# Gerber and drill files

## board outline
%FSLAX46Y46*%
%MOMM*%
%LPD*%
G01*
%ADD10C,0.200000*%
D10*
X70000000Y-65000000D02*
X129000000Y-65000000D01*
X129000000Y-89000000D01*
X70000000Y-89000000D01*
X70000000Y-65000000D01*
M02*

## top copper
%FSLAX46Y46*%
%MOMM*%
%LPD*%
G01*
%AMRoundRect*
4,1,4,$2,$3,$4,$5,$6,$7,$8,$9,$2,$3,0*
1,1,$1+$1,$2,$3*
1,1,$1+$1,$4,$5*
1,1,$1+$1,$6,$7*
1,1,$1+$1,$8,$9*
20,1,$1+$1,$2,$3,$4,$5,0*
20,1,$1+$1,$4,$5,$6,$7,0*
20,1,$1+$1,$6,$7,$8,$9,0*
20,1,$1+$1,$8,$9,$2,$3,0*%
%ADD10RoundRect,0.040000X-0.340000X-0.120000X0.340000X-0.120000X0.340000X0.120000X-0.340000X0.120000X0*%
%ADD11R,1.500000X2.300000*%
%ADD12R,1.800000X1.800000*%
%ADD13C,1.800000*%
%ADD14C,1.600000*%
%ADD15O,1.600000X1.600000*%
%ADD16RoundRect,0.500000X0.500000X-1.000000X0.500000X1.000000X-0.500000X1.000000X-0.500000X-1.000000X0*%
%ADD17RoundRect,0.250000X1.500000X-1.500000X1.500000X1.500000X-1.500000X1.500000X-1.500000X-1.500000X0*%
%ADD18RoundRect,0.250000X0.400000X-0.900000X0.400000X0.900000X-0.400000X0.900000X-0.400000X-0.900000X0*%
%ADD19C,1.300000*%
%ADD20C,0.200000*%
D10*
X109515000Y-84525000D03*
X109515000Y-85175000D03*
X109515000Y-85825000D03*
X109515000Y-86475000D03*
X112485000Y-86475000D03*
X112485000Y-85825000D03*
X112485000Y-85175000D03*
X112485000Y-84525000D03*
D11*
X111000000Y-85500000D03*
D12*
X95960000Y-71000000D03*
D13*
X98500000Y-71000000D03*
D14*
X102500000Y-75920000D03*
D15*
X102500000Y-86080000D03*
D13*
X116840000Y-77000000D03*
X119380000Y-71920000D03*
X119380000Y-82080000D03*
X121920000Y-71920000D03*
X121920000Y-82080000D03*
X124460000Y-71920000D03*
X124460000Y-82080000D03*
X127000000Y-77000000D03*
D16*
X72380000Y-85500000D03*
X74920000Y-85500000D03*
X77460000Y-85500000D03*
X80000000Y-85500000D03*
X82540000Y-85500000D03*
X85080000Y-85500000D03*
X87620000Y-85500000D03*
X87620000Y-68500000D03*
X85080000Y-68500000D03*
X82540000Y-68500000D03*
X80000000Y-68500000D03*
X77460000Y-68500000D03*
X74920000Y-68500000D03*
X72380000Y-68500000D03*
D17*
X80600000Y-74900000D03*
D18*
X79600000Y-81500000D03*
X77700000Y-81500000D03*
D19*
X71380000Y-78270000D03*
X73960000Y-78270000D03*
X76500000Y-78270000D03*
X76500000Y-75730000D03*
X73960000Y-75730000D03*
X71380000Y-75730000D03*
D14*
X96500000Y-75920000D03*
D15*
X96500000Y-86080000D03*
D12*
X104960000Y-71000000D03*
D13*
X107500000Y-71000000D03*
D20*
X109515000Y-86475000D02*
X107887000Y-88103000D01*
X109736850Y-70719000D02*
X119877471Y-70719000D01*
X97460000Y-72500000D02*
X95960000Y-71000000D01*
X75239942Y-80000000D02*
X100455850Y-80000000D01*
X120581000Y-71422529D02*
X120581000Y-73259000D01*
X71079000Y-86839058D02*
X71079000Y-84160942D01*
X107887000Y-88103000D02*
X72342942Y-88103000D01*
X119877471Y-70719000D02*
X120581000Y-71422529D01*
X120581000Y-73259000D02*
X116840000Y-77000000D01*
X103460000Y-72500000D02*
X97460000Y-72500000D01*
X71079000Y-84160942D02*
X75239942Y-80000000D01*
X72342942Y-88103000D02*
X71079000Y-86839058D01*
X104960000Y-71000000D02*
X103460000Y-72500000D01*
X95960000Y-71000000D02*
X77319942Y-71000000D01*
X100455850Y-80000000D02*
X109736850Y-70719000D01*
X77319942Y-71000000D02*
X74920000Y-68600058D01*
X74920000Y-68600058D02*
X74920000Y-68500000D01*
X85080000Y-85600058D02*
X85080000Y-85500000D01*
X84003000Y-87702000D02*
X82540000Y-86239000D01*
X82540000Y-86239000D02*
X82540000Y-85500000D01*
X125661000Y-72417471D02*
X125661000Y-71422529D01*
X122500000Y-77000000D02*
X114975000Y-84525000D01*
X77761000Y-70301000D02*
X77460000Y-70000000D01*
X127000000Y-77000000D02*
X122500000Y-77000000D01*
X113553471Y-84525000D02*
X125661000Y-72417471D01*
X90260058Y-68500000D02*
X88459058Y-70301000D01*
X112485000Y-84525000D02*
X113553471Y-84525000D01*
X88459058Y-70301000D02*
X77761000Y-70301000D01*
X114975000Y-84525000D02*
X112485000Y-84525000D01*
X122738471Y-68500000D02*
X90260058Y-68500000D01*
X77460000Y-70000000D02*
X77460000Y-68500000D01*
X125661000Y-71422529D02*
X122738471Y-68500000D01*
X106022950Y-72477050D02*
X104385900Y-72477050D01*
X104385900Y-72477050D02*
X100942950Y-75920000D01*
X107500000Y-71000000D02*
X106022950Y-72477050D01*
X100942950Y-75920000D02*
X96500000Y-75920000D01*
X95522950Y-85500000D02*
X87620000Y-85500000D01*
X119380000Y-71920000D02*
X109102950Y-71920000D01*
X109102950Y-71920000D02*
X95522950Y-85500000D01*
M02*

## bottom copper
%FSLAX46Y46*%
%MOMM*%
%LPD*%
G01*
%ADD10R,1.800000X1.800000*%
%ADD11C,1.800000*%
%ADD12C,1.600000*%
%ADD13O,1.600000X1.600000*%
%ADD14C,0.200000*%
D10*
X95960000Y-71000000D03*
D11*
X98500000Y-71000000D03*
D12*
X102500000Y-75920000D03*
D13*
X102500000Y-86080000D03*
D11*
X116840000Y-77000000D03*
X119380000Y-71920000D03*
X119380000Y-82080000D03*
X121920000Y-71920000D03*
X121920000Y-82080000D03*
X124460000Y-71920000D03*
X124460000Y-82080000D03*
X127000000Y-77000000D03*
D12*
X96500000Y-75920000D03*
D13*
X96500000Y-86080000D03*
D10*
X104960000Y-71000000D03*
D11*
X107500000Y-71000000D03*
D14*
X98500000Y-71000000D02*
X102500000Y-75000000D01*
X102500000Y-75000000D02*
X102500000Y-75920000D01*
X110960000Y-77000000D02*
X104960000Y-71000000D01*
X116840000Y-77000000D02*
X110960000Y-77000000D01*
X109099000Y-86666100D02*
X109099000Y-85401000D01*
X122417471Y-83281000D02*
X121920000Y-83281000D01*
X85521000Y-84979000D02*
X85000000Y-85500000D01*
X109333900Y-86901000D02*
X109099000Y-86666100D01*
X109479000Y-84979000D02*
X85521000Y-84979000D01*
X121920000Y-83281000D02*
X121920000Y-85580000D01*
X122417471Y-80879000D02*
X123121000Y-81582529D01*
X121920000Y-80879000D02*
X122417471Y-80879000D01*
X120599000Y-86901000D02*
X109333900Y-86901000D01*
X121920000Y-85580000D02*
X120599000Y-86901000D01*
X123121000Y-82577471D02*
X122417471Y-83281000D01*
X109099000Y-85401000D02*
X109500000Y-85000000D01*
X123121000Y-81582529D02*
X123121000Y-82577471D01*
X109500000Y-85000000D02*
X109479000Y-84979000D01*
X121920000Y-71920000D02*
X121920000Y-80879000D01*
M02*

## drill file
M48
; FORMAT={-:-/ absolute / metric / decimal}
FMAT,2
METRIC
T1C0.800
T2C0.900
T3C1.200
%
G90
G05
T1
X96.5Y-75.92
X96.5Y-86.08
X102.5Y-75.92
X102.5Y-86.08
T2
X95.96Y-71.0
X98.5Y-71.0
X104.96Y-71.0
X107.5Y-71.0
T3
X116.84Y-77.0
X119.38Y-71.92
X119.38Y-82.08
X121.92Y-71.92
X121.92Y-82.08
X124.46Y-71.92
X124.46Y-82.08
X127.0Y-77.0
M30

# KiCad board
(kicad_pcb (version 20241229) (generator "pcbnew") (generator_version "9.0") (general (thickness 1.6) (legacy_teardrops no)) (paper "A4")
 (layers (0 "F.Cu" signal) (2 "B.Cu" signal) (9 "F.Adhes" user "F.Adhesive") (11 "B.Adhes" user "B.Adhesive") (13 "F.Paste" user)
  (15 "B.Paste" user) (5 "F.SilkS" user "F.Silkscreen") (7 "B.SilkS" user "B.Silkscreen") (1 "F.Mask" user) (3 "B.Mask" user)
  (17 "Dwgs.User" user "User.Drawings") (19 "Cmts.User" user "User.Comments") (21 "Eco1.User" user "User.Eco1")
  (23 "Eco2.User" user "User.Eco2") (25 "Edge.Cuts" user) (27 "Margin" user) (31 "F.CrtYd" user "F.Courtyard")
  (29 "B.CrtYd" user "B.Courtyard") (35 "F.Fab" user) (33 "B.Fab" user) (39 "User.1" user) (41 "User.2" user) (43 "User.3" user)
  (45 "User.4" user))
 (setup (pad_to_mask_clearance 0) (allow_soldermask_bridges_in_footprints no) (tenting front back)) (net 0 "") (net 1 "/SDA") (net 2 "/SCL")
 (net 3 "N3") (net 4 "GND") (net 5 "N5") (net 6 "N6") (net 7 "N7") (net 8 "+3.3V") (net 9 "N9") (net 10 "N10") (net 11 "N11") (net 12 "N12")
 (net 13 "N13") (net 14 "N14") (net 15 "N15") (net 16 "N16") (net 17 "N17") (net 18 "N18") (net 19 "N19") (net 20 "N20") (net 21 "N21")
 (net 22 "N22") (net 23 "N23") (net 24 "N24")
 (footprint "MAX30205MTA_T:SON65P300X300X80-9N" (layer "F.Cu") (at 111 85.5)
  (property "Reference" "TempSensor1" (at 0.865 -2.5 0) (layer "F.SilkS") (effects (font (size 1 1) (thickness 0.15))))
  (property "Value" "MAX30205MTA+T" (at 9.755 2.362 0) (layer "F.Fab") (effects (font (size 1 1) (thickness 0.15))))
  (pad "1" smd roundrect (at -1.485 -0.975) (size 0.76 0.32) (layers "F.Cu" "F.Mask" "F.Paste") (roundrect_rratio 0.125) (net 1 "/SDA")
   (solder_mask_margin 0.102))
  (pad "2" smd roundrect (at -1.485 -0.325) (size 0.76 0.32) (layers "F.Cu" "F.Mask" "F.Paste") (roundrect_rratio 0.125) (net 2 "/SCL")
   (solder_mask_margin 0.102))
  (pad "3" smd roundrect (at -1.485 0.325) (size 0.76 0.32) (layers "F.Cu" "F.Mask" "F.Paste") (roundrect_rratio 0.125) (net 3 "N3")
   (solder_mask_margin 0.102))
  (pad "4" smd roundrect (at -1.485 0.975) (size 0.76 0.32) (layers "F.Cu" "F.Mask" "F.Paste") (roundrect_rratio 0.125) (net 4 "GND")
   (solder_mask_margin 0.102))
  (pad "5" smd roundrect (at 1.485 0.975) (size 0.76 0.32) (layers "F.Cu" "F.Mask" "F.Paste") (roundrect_rratio 0.125) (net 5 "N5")
   (solder_mask_margin 0.102))
  (pad "6" smd roundrect (at 1.485 0.325) (size 0.76 0.32) (layers "F.Cu" "F.Mask" "F.Paste") (roundrect_rratio 0.125) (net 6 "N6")
   (solder_mask_margin 0.102))
  (pad "7" smd roundrect (at 1.485 -0.325) (size 0.76 0.32) (layers "F.Cu" "F.Mask" "F.Paste") (roundrect_rratio 0.125) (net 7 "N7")
   (solder_mask_margin 0.102))
  (pad "8" smd roundrect (at 1.485 -0.975) (size 0.76 0.32) (layers "F.Cu" "F.Mask" "F.Paste") (roundrect_rratio 0.125) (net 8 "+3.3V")
   (solder_mask_margin 0.102))
  (pad "9" smd rect (at 0 0) (size 1.5 2.3) (layers "F.Cu" "F.Mask") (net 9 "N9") (solder_mask_margin 0.102)))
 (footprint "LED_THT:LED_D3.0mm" (layer "F.Cu") (at 95.96 71)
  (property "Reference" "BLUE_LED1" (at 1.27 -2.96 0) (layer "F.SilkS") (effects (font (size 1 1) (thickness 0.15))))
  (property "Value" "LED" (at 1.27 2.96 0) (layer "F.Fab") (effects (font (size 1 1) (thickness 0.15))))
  (pad "1" thru_hole rect (at 0 0) (size 1.8 1.8) (drill 0.9) (layers "*.Cu" "*.Mask") (remove_unused_layers no) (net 4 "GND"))
  (pad "2" thru_hole circle (at 2.54 0) (size 1.8 1.8) (drill 0.9) (layers "*.Cu" "*.Mask") (remove_unused_layers no) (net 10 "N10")))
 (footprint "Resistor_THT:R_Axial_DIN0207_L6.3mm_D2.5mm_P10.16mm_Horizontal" (layer "F.Cu") (at 102.5 75.92 -90)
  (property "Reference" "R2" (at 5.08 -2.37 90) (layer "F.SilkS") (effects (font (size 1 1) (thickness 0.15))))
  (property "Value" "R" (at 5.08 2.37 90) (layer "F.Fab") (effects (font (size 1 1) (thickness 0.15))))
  (pad "1" thru_hole circle (at 0 0 270) (size 1.6 1.6) (drill 0.8) (layers "*.Cu" "*.Mask") (remove_unused_layers no) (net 10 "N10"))
  (pad "2" thru_hole oval (at 10.16 0 270) (size 1.6 1.6) (drill 0.8) (layers "*.Cu" "*.Mask") (remove_unused_layers no) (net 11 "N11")))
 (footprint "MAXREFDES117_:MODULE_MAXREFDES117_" (layer "F.Cu") (at 121.92 77)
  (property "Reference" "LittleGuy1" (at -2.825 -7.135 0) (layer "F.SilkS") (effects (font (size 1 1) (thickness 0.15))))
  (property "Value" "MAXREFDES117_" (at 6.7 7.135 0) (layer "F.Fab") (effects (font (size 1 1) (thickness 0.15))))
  (pad "GND" thru_hole circle (at -5.08 0) (size 1.8 1.8) (drill 1.2) (layers "*.Cu" "*.Mask") (remove_unused_layers no) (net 4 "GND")
   (solder_mask_margin 0.102))
  (pad "INT" thru_hole circle (at -2.54 -5.08) (size 1.8 1.8) (drill 1.2) (layers "*.Cu" "*.Mask") (remove_unused_layers no) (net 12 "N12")
   (solder_mask_margin 0.102))
  (pad "INT1" thru_hole circle (at -2.54 5.08) (size 1.8 1.8) (drill 1.2) (layers "*.Cu" "*.Mask") (remove_unused_layers no) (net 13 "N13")
   (solder_mask_margin 0.102))
  (pad "SCL" thru_hole circle (at 0 -5.08) (size 1.8 1.8) (drill 1.2) (layers "*.Cu" "*.Mask") (remove_unused_layers no) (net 2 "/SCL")
   (solder_mask_margin 0.102))
  (pad "SCL1" thru_hole circle (at 0 5.08) (size 1.8 1.8) (drill 1.2) (layers "*.Cu" "*.Mask") (remove_unused_layers no) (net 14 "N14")
   (solder_mask_margin 0.102))
  (pad "SDA" thru_hole circle (at 2.54 -5.08) (size 1.8 1.8) (drill 1.2) (layers "*.Cu" "*.Mask") (remove_unused_layers no) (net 1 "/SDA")
   (solder_mask_margin 0.102))
  (pad "SDA1" thru_hole circle (at 2.54 5.08) (size 1.8 1.8) (drill 1.2) (layers "*.Cu" "*.Mask") (remove_unused_layers no) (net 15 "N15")
   (solder_mask_margin 0.102))
  (pad "VIN" thru_hole circle (at 5.08 0) (size 1.8 1.8) (drill 1.2) (layers "*.Cu" "*.Mask") (remove_unused_layers no) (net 8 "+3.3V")
   (solder_mask_margin 0.102)))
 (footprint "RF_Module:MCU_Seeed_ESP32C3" (layer "F.Cu") (at 80 77 90)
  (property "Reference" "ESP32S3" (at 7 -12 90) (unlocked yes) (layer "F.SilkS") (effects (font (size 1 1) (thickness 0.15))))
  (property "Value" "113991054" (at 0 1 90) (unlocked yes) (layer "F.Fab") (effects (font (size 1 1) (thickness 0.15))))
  (pad "" smd roundrect (at 1.1 -0.4 90) (size 1.5 1.5) (layers "F.Paste") (roundrect_rratio 0.1666666667))
  (pad "" smd roundrect (at 1.1 1.6 90) (size 1.5 1.5) (layers "F.Paste") (roundrect_rratio 0.1666666667))
  (pad "" smd roundrect (at 3.1 -0.4 90) (size 1.5 1.5) (layers "F.Paste") (roundrect_rratio 0.1666666667))
  (pad "" smd roundrect (at 3.1 1.6 90) (size 1.5 1.5) (layers "F.Paste") (roundrect_rratio 0.1666666667))
  (pad "1" smd roundrect (at -8.5 -7.62 90) (size 3 2) (layers "F.Cu" "F.Mask" "F.Paste") (roundrect_rratio 0.25) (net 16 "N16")
   (thermal_bridge_angle 45))
  (pad "2" smd roundrect (at -8.5 -5.08 90) (size 3 2) (layers "F.Cu" "F.Mask" "F.Paste") (roundrect_rratio 0.25) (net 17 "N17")
   (thermal_bridge_angle 45))
  (pad "3" smd roundrect (at -8.5 -2.54 90) (size 3 2) (layers "F.Cu" "F.Mask" "F.Paste") (roundrect_rratio 0.25) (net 11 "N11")
   (thermal_bridge_angle 45))
  (pad "4" smd roundrect (at -8.5 0 90) (size 3 2) (layers "F.Cu" "F.Mask" "F.Paste") (roundrect_rratio 0.25) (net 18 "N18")
   (thermal_bridge_angle 45))
  (pad "5" smd roundrect (at -8.5 2.54 90) (size 3 2) (layers "F.Cu" "F.Mask" "F.Paste") (roundrect_rratio 0.25) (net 1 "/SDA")
   (thermal_bridge_angle 45))
  (pad "6" smd roundrect (at -8.5 5.08 90) (size 3 2) (layers "F.Cu" "F.Mask" "F.Paste") (roundrect_rratio 0.25) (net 2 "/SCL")
   (thermal_bridge_angle 45))
  (pad "7" smd roundrect (at -8.5 7.62 90) (size 3 2) (layers "F.Cu" "F.Mask" "F.Paste") (roundrect_rratio 0.25) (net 12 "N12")
   (thermal_bridge_angle 45))
  (pad "8" smd roundrect (at 8.5 7.62 90) (size 3 2) (layers "F.Cu" "F.Mask" "F.Paste") (roundrect_rratio 0.25) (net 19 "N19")
   (thermal_bridge_angle 45))
  (pad "9" smd roundrect (at 8.5 5.08 90) (size 3 2) (layers "F.Cu" "F.Mask" "F.Paste") (roundrect_rratio 0.25) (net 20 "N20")
   (thermal_bridge_angle 45))
  (pad "10" smd roundrect (at 8.5 2.54 90) (size 3 2) (layers "F.Cu" "F.Mask" "F.Paste") (roundrect_rratio 0.25) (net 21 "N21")
   (thermal_bridge_angle 45))
  (pad "11" smd roundrect (at 8.5 0 90) (size 3 2) (layers "F.Cu" "F.Mask" "F.Paste") (roundrect_rratio 0.25) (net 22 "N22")
   (thermal_bridge_angle 45))
  (pad "12" smd roundrect (at 8.5 -2.54 90) (size 3 2) (layers "F.Cu" "F.Mask" "F.Paste") (roundrect_rratio 0.25) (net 8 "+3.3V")
   (thermal_bridge_angle 45))
  (pad "13" smd roundrect (at 8.5 -5.08 90) (size 3 2) (layers "F.Cu" "F.Mask" "F.Paste") (roundrect_rratio 0.25) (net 4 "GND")
   (thermal_bridge_angle 45))
  (pad "14" smd roundrect (at 8.5 -7.62 90) (size 3 2) (layers "F.Cu" "F.Mask" "F.Paste") (roundrect_rratio 0.25) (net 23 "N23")
   (thermal_bridge_angle 45))
  (pad "15" smd roundrect (at 2.1 0.6 90) (size 3.5 3.5) (layers "F.Cu" "F.Mask") (roundrect_rratio 0.07142857143))
  (pad "16" smd roundrect (at -4.5 -0.4 90) (size 2.3 1.3) (layers "F.Cu" "F.Mask" "F.Paste") (roundrect_rratio 0.1923076923))
  (pad "17" smd roundrect (at -4.5 -2.3 90) (size 2.3 1.3) (layers "F.Cu" "F.Mask" "F.Paste") (roundrect_rratio 0.1923076923))
  (pad "18" smd circle (at -1.27 -8.62 90) (size 1.3 1.3) (layers "F.Cu" "F.Mask" "F.Paste"))
  (pad "19" smd circle (at -1.27 -6.04 90) (size 1.3 1.3) (layers "F.Cu" "F.Mask" "F.Paste"))
  (pad "20" smd circle (at -1.27 -3.5 90) (size 1.3 1.3) (layers "F.Cu" "F.Mask" "F.Paste"))
  (pad "21" smd circle (at 1.27 -3.5 90) (size 1.3 1.3) (layers "F.Cu" "F.Mask" "F.Paste"))
  (pad "22" smd circle (at 1.27 -6.04 90) (size 1.3 1.3) (layers "F.Cu" "F.Mask" "F.Paste"))
  (pad "23" smd circle (at 1.27 -8.62 90) (size 1.3 1.3) (layers "F.Cu" "F.Mask" "F.Paste")))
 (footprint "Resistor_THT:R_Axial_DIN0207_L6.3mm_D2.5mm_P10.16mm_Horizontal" (layer "F.Cu") (at 96.5 75.92 -90)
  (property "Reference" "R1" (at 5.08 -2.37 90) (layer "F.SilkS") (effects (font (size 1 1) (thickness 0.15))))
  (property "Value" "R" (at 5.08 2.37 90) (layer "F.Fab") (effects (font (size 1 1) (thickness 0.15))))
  (pad "1" thru_hole circle (at 0 0 270) (size 1.6 1.6) (drill 0.8) (layers "*.Cu" "*.Mask") (remove_unused_layers no) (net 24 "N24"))
  (pad "2" thru_hole oval (at 10.16 0 270) (size 1.6 1.6) (drill 0.8) (layers "*.Cu" "*.Mask") (remove_unused_layers no) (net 17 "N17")))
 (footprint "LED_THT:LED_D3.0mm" (layer "F.Cu") (at 104.96 71)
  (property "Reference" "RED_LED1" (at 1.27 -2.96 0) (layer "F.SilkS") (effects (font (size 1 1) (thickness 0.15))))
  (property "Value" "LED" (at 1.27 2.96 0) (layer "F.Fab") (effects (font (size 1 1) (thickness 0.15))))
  (pad "1" thru_hole rect (at 0 0) (size 1.8 1.8) (drill 0.9) (layers "*.Cu" "*.Mask") (remove_unused_layers no) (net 4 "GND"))
  (pad "2" thru_hole circle (at 2.54 0) (size 1.8 1.8) (drill 0.9) (layers "*.Cu" "*.Mask") (remove_unused_layers no) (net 24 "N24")))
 (gr_rect (start 70 65) (end 129 89) (stroke (width 0.2) (type solid)) (fill no) (layer "Edge.Cuts"))
 (segment (start 98.5 71) (end 102.5 75) (width 0.2) (layer "B.Cu") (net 10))
 (segment (start 102.5 75) (end 102.5 75.92) (width 0.2) (layer "B.Cu") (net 10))
 (segment (start 109.515 86.475) (end 107.887 88.103) (width 0.2) (layer "F.Cu") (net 4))
 (segment (start 109.73685 70.719) (end 119.877471 70.719) (width 0.2) (layer "F.Cu") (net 4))
 (segment (start 97.46 72.5) (end 95.96 71) (width 0.2) (layer "F.Cu") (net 4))
 (segment (start 75.239942 80) (end 100.45585 80) (width 0.2) (layer "F.Cu") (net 4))
 (segment (start 120.581 71.422529) (end 120.581 73.259) (width 0.2) (layer "F.Cu") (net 4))
 (segment (start 71.079 86.839058) (end 71.079 84.160942) (width 0.2) (layer "F.Cu") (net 4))
 (segment (start 107.887 88.103) (end 72.342942 88.103) (width 0.2) (layer "F.Cu") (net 4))
 (segment (start 119.877471 70.719) (end 120.581 71.422529) (width 0.2) (layer "F.Cu") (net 4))
 (segment (start 120.581 73.259) (end 116.84 77) (width 0.2) (layer "F.Cu") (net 4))
 (segment (start 103.46 72.5) (end 97.46 72.5) (width 0.2) (layer "F.Cu") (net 4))
 (segment (start 71.079 84.160942) (end 75.239942 80) (width 0.2) (layer "F.Cu") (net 4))
 (segment (start 72.342942 88.103) (end 71.079 86.839058) (width 0.2) (layer "F.Cu") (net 4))
 (segment (start 104.96 71) (end 103.46 72.5) (width 0.2) (layer "F.Cu") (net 4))
 (segment (start 95.96 71) (end 77.319942 71) (width 0.2) (layer "F.Cu") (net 4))
 (segment (start 100.45585 80) (end 109.73685 70.719) (width 0.2) (layer "F.Cu") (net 4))
 (segment (start 77.319942 71) (end 74.92 68.600058) (width 0.2) (layer "F.Cu") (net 4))
 (segment (start 74.92 68.600058) (end 74.92 68.5) (width 0.2) (layer "F.Cu") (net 4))
 (segment (start 110.96 77) (end 104.96 71) (width 0.2) (layer "B.Cu") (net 4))
 (segment (start 116.84 77) (end 110.96 77) (width 0.2) (layer "B.Cu") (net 4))
 (segment (start 85.08 85.600058) (end 85.08 85.5) (width 0.2) (layer "F.Cu") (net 2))
 (segment (start 109.099 86.6661) (end 109.099 85.401) (width 0.2) (layer "B.Cu") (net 2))
 (segment (start 122.417471 83.281) (end 121.92 83.281) (width 0.2) (layer "B.Cu") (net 2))
 (segment (start 85.521 84.979) (end 85 85.5) (width 0.2) (layer "B.Cu") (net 2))
 (segment (start 109.3339 86.901) (end 109.099 86.6661) (width 0.2) (layer "B.Cu") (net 2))
 (segment (start 109.479 84.979) (end 85.521 84.979) (width 0.2) (layer "B.Cu") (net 2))
 (segment (start 121.92 83.281) (end 121.92 85.58) (width 0.2) (layer "B.Cu") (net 2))
 (segment (start 122.417471 80.879) (end 123.121 81.582529) (width 0.2) (layer "B.Cu") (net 2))
 (segment (start 121.92 80.879) (end 122.417471 80.879) (width 0.2) (layer "B.Cu") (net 2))
 (segment (start 120.599 86.901) (end 109.3339 86.901) (width 0.2) (layer "B.Cu") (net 2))
 (segment (start 121.92 85.58) (end 120.599 86.901) (width 0.2) (layer "B.Cu") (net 2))
 (segment (start 123.121 82.577471) (end 122.417471 83.281) (width 0.2) (layer "B.Cu") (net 2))
 (segment (start 109.099 85.401) (end 109.5 85) (width 0.2) (layer "B.Cu") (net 2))
 (segment (start 123.121 81.582529) (end 123.121 82.577471) (width 0.2) (layer "B.Cu") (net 2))
 (segment (start 109.5 85) (end 109.479 84.979) (width 0.2) (layer "B.Cu") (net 2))
 (segment (start 121.92 71.92) (end 121.92 80.879) (width 0.2) (layer "B.Cu") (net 2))
 (segment (start 84.003 87.702) (end 82.54 86.239) (width 0.2) (layer "F.Cu") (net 1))
 (segment (start 82.54 86.239) (end 82.54 85.5) (width 0.2) (layer "F.Cu") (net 1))
 (segment (start 125.661 72.417471) (end 125.661 71.422529) (width 0.2) (layer "F.Cu") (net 8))
 (segment (start 122.5 77) (end 114.975 84.525) (width 0.2) (layer "F.Cu") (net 8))
 (segment (start 77.761 70.301) (end 77.46 70) (width 0.2) (layer "F.Cu") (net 8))
 (segment (start 127 77) (end 122.5 77) (width 0.2) (layer "F.Cu") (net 8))
 (segment (start 113.553471 84.525) (end 125.661 72.417471) (width 0.2) (layer "F.Cu") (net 8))
 (segment (start 90.260058 68.5) (end 88.459058 70.301) (width 0.2) (layer "F.Cu") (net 8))
 (segment (start 112.485 84.525) (end 113.553471 84.525) (width 0.2) (layer "F.Cu") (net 8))
 (segment (start 88.459058 70.301) (end 77.761 70.301) (width 0.2) (layer "F.Cu") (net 8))
 (segment (start 114.975 84.525) (end 112.485 84.525) (width 0.2) (layer "F.Cu") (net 8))
 (segment (start 122.738471 68.5) (end 90.260058 68.5) (width 0.2) (layer "F.Cu") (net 8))
 (segment (start 77.46 70) (end 77.46 68.5) (width 0.2) (layer "F.Cu") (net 8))
 (segment (start 125.661 71.422529) (end 122.738471 68.5) (width 0.2) (layer "F.Cu") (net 8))
 (segment (start 106.02295 72.47705) (end 104.3859 72.47705) (width 0.2) (layer "F.Cu") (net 24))
 (segment (start 104.3859 72.47705) (end 100.94295 75.92) (width 0.2) (layer "F.Cu") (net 24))
 (segment (start 107.5 71) (end 106.02295 72.47705) (width 0.2) (layer "F.Cu") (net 24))
 (segment (start 100.94295 75.92) (end 96.5 75.92) (width 0.2) (layer "F.Cu") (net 24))
 (segment (start 95.52295 85.5) (end 87.62 85.5) (width 0.2) (layer "F.Cu") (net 12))
 (segment (start 119.38 71.92) (end 109.10295 71.92) (width 0.2) (layer "F.Cu") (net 12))
 (segment (start 109.10295 71.92) (end 95.52295 85.5) (width 0.2) (layer "F.Cu") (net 12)))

